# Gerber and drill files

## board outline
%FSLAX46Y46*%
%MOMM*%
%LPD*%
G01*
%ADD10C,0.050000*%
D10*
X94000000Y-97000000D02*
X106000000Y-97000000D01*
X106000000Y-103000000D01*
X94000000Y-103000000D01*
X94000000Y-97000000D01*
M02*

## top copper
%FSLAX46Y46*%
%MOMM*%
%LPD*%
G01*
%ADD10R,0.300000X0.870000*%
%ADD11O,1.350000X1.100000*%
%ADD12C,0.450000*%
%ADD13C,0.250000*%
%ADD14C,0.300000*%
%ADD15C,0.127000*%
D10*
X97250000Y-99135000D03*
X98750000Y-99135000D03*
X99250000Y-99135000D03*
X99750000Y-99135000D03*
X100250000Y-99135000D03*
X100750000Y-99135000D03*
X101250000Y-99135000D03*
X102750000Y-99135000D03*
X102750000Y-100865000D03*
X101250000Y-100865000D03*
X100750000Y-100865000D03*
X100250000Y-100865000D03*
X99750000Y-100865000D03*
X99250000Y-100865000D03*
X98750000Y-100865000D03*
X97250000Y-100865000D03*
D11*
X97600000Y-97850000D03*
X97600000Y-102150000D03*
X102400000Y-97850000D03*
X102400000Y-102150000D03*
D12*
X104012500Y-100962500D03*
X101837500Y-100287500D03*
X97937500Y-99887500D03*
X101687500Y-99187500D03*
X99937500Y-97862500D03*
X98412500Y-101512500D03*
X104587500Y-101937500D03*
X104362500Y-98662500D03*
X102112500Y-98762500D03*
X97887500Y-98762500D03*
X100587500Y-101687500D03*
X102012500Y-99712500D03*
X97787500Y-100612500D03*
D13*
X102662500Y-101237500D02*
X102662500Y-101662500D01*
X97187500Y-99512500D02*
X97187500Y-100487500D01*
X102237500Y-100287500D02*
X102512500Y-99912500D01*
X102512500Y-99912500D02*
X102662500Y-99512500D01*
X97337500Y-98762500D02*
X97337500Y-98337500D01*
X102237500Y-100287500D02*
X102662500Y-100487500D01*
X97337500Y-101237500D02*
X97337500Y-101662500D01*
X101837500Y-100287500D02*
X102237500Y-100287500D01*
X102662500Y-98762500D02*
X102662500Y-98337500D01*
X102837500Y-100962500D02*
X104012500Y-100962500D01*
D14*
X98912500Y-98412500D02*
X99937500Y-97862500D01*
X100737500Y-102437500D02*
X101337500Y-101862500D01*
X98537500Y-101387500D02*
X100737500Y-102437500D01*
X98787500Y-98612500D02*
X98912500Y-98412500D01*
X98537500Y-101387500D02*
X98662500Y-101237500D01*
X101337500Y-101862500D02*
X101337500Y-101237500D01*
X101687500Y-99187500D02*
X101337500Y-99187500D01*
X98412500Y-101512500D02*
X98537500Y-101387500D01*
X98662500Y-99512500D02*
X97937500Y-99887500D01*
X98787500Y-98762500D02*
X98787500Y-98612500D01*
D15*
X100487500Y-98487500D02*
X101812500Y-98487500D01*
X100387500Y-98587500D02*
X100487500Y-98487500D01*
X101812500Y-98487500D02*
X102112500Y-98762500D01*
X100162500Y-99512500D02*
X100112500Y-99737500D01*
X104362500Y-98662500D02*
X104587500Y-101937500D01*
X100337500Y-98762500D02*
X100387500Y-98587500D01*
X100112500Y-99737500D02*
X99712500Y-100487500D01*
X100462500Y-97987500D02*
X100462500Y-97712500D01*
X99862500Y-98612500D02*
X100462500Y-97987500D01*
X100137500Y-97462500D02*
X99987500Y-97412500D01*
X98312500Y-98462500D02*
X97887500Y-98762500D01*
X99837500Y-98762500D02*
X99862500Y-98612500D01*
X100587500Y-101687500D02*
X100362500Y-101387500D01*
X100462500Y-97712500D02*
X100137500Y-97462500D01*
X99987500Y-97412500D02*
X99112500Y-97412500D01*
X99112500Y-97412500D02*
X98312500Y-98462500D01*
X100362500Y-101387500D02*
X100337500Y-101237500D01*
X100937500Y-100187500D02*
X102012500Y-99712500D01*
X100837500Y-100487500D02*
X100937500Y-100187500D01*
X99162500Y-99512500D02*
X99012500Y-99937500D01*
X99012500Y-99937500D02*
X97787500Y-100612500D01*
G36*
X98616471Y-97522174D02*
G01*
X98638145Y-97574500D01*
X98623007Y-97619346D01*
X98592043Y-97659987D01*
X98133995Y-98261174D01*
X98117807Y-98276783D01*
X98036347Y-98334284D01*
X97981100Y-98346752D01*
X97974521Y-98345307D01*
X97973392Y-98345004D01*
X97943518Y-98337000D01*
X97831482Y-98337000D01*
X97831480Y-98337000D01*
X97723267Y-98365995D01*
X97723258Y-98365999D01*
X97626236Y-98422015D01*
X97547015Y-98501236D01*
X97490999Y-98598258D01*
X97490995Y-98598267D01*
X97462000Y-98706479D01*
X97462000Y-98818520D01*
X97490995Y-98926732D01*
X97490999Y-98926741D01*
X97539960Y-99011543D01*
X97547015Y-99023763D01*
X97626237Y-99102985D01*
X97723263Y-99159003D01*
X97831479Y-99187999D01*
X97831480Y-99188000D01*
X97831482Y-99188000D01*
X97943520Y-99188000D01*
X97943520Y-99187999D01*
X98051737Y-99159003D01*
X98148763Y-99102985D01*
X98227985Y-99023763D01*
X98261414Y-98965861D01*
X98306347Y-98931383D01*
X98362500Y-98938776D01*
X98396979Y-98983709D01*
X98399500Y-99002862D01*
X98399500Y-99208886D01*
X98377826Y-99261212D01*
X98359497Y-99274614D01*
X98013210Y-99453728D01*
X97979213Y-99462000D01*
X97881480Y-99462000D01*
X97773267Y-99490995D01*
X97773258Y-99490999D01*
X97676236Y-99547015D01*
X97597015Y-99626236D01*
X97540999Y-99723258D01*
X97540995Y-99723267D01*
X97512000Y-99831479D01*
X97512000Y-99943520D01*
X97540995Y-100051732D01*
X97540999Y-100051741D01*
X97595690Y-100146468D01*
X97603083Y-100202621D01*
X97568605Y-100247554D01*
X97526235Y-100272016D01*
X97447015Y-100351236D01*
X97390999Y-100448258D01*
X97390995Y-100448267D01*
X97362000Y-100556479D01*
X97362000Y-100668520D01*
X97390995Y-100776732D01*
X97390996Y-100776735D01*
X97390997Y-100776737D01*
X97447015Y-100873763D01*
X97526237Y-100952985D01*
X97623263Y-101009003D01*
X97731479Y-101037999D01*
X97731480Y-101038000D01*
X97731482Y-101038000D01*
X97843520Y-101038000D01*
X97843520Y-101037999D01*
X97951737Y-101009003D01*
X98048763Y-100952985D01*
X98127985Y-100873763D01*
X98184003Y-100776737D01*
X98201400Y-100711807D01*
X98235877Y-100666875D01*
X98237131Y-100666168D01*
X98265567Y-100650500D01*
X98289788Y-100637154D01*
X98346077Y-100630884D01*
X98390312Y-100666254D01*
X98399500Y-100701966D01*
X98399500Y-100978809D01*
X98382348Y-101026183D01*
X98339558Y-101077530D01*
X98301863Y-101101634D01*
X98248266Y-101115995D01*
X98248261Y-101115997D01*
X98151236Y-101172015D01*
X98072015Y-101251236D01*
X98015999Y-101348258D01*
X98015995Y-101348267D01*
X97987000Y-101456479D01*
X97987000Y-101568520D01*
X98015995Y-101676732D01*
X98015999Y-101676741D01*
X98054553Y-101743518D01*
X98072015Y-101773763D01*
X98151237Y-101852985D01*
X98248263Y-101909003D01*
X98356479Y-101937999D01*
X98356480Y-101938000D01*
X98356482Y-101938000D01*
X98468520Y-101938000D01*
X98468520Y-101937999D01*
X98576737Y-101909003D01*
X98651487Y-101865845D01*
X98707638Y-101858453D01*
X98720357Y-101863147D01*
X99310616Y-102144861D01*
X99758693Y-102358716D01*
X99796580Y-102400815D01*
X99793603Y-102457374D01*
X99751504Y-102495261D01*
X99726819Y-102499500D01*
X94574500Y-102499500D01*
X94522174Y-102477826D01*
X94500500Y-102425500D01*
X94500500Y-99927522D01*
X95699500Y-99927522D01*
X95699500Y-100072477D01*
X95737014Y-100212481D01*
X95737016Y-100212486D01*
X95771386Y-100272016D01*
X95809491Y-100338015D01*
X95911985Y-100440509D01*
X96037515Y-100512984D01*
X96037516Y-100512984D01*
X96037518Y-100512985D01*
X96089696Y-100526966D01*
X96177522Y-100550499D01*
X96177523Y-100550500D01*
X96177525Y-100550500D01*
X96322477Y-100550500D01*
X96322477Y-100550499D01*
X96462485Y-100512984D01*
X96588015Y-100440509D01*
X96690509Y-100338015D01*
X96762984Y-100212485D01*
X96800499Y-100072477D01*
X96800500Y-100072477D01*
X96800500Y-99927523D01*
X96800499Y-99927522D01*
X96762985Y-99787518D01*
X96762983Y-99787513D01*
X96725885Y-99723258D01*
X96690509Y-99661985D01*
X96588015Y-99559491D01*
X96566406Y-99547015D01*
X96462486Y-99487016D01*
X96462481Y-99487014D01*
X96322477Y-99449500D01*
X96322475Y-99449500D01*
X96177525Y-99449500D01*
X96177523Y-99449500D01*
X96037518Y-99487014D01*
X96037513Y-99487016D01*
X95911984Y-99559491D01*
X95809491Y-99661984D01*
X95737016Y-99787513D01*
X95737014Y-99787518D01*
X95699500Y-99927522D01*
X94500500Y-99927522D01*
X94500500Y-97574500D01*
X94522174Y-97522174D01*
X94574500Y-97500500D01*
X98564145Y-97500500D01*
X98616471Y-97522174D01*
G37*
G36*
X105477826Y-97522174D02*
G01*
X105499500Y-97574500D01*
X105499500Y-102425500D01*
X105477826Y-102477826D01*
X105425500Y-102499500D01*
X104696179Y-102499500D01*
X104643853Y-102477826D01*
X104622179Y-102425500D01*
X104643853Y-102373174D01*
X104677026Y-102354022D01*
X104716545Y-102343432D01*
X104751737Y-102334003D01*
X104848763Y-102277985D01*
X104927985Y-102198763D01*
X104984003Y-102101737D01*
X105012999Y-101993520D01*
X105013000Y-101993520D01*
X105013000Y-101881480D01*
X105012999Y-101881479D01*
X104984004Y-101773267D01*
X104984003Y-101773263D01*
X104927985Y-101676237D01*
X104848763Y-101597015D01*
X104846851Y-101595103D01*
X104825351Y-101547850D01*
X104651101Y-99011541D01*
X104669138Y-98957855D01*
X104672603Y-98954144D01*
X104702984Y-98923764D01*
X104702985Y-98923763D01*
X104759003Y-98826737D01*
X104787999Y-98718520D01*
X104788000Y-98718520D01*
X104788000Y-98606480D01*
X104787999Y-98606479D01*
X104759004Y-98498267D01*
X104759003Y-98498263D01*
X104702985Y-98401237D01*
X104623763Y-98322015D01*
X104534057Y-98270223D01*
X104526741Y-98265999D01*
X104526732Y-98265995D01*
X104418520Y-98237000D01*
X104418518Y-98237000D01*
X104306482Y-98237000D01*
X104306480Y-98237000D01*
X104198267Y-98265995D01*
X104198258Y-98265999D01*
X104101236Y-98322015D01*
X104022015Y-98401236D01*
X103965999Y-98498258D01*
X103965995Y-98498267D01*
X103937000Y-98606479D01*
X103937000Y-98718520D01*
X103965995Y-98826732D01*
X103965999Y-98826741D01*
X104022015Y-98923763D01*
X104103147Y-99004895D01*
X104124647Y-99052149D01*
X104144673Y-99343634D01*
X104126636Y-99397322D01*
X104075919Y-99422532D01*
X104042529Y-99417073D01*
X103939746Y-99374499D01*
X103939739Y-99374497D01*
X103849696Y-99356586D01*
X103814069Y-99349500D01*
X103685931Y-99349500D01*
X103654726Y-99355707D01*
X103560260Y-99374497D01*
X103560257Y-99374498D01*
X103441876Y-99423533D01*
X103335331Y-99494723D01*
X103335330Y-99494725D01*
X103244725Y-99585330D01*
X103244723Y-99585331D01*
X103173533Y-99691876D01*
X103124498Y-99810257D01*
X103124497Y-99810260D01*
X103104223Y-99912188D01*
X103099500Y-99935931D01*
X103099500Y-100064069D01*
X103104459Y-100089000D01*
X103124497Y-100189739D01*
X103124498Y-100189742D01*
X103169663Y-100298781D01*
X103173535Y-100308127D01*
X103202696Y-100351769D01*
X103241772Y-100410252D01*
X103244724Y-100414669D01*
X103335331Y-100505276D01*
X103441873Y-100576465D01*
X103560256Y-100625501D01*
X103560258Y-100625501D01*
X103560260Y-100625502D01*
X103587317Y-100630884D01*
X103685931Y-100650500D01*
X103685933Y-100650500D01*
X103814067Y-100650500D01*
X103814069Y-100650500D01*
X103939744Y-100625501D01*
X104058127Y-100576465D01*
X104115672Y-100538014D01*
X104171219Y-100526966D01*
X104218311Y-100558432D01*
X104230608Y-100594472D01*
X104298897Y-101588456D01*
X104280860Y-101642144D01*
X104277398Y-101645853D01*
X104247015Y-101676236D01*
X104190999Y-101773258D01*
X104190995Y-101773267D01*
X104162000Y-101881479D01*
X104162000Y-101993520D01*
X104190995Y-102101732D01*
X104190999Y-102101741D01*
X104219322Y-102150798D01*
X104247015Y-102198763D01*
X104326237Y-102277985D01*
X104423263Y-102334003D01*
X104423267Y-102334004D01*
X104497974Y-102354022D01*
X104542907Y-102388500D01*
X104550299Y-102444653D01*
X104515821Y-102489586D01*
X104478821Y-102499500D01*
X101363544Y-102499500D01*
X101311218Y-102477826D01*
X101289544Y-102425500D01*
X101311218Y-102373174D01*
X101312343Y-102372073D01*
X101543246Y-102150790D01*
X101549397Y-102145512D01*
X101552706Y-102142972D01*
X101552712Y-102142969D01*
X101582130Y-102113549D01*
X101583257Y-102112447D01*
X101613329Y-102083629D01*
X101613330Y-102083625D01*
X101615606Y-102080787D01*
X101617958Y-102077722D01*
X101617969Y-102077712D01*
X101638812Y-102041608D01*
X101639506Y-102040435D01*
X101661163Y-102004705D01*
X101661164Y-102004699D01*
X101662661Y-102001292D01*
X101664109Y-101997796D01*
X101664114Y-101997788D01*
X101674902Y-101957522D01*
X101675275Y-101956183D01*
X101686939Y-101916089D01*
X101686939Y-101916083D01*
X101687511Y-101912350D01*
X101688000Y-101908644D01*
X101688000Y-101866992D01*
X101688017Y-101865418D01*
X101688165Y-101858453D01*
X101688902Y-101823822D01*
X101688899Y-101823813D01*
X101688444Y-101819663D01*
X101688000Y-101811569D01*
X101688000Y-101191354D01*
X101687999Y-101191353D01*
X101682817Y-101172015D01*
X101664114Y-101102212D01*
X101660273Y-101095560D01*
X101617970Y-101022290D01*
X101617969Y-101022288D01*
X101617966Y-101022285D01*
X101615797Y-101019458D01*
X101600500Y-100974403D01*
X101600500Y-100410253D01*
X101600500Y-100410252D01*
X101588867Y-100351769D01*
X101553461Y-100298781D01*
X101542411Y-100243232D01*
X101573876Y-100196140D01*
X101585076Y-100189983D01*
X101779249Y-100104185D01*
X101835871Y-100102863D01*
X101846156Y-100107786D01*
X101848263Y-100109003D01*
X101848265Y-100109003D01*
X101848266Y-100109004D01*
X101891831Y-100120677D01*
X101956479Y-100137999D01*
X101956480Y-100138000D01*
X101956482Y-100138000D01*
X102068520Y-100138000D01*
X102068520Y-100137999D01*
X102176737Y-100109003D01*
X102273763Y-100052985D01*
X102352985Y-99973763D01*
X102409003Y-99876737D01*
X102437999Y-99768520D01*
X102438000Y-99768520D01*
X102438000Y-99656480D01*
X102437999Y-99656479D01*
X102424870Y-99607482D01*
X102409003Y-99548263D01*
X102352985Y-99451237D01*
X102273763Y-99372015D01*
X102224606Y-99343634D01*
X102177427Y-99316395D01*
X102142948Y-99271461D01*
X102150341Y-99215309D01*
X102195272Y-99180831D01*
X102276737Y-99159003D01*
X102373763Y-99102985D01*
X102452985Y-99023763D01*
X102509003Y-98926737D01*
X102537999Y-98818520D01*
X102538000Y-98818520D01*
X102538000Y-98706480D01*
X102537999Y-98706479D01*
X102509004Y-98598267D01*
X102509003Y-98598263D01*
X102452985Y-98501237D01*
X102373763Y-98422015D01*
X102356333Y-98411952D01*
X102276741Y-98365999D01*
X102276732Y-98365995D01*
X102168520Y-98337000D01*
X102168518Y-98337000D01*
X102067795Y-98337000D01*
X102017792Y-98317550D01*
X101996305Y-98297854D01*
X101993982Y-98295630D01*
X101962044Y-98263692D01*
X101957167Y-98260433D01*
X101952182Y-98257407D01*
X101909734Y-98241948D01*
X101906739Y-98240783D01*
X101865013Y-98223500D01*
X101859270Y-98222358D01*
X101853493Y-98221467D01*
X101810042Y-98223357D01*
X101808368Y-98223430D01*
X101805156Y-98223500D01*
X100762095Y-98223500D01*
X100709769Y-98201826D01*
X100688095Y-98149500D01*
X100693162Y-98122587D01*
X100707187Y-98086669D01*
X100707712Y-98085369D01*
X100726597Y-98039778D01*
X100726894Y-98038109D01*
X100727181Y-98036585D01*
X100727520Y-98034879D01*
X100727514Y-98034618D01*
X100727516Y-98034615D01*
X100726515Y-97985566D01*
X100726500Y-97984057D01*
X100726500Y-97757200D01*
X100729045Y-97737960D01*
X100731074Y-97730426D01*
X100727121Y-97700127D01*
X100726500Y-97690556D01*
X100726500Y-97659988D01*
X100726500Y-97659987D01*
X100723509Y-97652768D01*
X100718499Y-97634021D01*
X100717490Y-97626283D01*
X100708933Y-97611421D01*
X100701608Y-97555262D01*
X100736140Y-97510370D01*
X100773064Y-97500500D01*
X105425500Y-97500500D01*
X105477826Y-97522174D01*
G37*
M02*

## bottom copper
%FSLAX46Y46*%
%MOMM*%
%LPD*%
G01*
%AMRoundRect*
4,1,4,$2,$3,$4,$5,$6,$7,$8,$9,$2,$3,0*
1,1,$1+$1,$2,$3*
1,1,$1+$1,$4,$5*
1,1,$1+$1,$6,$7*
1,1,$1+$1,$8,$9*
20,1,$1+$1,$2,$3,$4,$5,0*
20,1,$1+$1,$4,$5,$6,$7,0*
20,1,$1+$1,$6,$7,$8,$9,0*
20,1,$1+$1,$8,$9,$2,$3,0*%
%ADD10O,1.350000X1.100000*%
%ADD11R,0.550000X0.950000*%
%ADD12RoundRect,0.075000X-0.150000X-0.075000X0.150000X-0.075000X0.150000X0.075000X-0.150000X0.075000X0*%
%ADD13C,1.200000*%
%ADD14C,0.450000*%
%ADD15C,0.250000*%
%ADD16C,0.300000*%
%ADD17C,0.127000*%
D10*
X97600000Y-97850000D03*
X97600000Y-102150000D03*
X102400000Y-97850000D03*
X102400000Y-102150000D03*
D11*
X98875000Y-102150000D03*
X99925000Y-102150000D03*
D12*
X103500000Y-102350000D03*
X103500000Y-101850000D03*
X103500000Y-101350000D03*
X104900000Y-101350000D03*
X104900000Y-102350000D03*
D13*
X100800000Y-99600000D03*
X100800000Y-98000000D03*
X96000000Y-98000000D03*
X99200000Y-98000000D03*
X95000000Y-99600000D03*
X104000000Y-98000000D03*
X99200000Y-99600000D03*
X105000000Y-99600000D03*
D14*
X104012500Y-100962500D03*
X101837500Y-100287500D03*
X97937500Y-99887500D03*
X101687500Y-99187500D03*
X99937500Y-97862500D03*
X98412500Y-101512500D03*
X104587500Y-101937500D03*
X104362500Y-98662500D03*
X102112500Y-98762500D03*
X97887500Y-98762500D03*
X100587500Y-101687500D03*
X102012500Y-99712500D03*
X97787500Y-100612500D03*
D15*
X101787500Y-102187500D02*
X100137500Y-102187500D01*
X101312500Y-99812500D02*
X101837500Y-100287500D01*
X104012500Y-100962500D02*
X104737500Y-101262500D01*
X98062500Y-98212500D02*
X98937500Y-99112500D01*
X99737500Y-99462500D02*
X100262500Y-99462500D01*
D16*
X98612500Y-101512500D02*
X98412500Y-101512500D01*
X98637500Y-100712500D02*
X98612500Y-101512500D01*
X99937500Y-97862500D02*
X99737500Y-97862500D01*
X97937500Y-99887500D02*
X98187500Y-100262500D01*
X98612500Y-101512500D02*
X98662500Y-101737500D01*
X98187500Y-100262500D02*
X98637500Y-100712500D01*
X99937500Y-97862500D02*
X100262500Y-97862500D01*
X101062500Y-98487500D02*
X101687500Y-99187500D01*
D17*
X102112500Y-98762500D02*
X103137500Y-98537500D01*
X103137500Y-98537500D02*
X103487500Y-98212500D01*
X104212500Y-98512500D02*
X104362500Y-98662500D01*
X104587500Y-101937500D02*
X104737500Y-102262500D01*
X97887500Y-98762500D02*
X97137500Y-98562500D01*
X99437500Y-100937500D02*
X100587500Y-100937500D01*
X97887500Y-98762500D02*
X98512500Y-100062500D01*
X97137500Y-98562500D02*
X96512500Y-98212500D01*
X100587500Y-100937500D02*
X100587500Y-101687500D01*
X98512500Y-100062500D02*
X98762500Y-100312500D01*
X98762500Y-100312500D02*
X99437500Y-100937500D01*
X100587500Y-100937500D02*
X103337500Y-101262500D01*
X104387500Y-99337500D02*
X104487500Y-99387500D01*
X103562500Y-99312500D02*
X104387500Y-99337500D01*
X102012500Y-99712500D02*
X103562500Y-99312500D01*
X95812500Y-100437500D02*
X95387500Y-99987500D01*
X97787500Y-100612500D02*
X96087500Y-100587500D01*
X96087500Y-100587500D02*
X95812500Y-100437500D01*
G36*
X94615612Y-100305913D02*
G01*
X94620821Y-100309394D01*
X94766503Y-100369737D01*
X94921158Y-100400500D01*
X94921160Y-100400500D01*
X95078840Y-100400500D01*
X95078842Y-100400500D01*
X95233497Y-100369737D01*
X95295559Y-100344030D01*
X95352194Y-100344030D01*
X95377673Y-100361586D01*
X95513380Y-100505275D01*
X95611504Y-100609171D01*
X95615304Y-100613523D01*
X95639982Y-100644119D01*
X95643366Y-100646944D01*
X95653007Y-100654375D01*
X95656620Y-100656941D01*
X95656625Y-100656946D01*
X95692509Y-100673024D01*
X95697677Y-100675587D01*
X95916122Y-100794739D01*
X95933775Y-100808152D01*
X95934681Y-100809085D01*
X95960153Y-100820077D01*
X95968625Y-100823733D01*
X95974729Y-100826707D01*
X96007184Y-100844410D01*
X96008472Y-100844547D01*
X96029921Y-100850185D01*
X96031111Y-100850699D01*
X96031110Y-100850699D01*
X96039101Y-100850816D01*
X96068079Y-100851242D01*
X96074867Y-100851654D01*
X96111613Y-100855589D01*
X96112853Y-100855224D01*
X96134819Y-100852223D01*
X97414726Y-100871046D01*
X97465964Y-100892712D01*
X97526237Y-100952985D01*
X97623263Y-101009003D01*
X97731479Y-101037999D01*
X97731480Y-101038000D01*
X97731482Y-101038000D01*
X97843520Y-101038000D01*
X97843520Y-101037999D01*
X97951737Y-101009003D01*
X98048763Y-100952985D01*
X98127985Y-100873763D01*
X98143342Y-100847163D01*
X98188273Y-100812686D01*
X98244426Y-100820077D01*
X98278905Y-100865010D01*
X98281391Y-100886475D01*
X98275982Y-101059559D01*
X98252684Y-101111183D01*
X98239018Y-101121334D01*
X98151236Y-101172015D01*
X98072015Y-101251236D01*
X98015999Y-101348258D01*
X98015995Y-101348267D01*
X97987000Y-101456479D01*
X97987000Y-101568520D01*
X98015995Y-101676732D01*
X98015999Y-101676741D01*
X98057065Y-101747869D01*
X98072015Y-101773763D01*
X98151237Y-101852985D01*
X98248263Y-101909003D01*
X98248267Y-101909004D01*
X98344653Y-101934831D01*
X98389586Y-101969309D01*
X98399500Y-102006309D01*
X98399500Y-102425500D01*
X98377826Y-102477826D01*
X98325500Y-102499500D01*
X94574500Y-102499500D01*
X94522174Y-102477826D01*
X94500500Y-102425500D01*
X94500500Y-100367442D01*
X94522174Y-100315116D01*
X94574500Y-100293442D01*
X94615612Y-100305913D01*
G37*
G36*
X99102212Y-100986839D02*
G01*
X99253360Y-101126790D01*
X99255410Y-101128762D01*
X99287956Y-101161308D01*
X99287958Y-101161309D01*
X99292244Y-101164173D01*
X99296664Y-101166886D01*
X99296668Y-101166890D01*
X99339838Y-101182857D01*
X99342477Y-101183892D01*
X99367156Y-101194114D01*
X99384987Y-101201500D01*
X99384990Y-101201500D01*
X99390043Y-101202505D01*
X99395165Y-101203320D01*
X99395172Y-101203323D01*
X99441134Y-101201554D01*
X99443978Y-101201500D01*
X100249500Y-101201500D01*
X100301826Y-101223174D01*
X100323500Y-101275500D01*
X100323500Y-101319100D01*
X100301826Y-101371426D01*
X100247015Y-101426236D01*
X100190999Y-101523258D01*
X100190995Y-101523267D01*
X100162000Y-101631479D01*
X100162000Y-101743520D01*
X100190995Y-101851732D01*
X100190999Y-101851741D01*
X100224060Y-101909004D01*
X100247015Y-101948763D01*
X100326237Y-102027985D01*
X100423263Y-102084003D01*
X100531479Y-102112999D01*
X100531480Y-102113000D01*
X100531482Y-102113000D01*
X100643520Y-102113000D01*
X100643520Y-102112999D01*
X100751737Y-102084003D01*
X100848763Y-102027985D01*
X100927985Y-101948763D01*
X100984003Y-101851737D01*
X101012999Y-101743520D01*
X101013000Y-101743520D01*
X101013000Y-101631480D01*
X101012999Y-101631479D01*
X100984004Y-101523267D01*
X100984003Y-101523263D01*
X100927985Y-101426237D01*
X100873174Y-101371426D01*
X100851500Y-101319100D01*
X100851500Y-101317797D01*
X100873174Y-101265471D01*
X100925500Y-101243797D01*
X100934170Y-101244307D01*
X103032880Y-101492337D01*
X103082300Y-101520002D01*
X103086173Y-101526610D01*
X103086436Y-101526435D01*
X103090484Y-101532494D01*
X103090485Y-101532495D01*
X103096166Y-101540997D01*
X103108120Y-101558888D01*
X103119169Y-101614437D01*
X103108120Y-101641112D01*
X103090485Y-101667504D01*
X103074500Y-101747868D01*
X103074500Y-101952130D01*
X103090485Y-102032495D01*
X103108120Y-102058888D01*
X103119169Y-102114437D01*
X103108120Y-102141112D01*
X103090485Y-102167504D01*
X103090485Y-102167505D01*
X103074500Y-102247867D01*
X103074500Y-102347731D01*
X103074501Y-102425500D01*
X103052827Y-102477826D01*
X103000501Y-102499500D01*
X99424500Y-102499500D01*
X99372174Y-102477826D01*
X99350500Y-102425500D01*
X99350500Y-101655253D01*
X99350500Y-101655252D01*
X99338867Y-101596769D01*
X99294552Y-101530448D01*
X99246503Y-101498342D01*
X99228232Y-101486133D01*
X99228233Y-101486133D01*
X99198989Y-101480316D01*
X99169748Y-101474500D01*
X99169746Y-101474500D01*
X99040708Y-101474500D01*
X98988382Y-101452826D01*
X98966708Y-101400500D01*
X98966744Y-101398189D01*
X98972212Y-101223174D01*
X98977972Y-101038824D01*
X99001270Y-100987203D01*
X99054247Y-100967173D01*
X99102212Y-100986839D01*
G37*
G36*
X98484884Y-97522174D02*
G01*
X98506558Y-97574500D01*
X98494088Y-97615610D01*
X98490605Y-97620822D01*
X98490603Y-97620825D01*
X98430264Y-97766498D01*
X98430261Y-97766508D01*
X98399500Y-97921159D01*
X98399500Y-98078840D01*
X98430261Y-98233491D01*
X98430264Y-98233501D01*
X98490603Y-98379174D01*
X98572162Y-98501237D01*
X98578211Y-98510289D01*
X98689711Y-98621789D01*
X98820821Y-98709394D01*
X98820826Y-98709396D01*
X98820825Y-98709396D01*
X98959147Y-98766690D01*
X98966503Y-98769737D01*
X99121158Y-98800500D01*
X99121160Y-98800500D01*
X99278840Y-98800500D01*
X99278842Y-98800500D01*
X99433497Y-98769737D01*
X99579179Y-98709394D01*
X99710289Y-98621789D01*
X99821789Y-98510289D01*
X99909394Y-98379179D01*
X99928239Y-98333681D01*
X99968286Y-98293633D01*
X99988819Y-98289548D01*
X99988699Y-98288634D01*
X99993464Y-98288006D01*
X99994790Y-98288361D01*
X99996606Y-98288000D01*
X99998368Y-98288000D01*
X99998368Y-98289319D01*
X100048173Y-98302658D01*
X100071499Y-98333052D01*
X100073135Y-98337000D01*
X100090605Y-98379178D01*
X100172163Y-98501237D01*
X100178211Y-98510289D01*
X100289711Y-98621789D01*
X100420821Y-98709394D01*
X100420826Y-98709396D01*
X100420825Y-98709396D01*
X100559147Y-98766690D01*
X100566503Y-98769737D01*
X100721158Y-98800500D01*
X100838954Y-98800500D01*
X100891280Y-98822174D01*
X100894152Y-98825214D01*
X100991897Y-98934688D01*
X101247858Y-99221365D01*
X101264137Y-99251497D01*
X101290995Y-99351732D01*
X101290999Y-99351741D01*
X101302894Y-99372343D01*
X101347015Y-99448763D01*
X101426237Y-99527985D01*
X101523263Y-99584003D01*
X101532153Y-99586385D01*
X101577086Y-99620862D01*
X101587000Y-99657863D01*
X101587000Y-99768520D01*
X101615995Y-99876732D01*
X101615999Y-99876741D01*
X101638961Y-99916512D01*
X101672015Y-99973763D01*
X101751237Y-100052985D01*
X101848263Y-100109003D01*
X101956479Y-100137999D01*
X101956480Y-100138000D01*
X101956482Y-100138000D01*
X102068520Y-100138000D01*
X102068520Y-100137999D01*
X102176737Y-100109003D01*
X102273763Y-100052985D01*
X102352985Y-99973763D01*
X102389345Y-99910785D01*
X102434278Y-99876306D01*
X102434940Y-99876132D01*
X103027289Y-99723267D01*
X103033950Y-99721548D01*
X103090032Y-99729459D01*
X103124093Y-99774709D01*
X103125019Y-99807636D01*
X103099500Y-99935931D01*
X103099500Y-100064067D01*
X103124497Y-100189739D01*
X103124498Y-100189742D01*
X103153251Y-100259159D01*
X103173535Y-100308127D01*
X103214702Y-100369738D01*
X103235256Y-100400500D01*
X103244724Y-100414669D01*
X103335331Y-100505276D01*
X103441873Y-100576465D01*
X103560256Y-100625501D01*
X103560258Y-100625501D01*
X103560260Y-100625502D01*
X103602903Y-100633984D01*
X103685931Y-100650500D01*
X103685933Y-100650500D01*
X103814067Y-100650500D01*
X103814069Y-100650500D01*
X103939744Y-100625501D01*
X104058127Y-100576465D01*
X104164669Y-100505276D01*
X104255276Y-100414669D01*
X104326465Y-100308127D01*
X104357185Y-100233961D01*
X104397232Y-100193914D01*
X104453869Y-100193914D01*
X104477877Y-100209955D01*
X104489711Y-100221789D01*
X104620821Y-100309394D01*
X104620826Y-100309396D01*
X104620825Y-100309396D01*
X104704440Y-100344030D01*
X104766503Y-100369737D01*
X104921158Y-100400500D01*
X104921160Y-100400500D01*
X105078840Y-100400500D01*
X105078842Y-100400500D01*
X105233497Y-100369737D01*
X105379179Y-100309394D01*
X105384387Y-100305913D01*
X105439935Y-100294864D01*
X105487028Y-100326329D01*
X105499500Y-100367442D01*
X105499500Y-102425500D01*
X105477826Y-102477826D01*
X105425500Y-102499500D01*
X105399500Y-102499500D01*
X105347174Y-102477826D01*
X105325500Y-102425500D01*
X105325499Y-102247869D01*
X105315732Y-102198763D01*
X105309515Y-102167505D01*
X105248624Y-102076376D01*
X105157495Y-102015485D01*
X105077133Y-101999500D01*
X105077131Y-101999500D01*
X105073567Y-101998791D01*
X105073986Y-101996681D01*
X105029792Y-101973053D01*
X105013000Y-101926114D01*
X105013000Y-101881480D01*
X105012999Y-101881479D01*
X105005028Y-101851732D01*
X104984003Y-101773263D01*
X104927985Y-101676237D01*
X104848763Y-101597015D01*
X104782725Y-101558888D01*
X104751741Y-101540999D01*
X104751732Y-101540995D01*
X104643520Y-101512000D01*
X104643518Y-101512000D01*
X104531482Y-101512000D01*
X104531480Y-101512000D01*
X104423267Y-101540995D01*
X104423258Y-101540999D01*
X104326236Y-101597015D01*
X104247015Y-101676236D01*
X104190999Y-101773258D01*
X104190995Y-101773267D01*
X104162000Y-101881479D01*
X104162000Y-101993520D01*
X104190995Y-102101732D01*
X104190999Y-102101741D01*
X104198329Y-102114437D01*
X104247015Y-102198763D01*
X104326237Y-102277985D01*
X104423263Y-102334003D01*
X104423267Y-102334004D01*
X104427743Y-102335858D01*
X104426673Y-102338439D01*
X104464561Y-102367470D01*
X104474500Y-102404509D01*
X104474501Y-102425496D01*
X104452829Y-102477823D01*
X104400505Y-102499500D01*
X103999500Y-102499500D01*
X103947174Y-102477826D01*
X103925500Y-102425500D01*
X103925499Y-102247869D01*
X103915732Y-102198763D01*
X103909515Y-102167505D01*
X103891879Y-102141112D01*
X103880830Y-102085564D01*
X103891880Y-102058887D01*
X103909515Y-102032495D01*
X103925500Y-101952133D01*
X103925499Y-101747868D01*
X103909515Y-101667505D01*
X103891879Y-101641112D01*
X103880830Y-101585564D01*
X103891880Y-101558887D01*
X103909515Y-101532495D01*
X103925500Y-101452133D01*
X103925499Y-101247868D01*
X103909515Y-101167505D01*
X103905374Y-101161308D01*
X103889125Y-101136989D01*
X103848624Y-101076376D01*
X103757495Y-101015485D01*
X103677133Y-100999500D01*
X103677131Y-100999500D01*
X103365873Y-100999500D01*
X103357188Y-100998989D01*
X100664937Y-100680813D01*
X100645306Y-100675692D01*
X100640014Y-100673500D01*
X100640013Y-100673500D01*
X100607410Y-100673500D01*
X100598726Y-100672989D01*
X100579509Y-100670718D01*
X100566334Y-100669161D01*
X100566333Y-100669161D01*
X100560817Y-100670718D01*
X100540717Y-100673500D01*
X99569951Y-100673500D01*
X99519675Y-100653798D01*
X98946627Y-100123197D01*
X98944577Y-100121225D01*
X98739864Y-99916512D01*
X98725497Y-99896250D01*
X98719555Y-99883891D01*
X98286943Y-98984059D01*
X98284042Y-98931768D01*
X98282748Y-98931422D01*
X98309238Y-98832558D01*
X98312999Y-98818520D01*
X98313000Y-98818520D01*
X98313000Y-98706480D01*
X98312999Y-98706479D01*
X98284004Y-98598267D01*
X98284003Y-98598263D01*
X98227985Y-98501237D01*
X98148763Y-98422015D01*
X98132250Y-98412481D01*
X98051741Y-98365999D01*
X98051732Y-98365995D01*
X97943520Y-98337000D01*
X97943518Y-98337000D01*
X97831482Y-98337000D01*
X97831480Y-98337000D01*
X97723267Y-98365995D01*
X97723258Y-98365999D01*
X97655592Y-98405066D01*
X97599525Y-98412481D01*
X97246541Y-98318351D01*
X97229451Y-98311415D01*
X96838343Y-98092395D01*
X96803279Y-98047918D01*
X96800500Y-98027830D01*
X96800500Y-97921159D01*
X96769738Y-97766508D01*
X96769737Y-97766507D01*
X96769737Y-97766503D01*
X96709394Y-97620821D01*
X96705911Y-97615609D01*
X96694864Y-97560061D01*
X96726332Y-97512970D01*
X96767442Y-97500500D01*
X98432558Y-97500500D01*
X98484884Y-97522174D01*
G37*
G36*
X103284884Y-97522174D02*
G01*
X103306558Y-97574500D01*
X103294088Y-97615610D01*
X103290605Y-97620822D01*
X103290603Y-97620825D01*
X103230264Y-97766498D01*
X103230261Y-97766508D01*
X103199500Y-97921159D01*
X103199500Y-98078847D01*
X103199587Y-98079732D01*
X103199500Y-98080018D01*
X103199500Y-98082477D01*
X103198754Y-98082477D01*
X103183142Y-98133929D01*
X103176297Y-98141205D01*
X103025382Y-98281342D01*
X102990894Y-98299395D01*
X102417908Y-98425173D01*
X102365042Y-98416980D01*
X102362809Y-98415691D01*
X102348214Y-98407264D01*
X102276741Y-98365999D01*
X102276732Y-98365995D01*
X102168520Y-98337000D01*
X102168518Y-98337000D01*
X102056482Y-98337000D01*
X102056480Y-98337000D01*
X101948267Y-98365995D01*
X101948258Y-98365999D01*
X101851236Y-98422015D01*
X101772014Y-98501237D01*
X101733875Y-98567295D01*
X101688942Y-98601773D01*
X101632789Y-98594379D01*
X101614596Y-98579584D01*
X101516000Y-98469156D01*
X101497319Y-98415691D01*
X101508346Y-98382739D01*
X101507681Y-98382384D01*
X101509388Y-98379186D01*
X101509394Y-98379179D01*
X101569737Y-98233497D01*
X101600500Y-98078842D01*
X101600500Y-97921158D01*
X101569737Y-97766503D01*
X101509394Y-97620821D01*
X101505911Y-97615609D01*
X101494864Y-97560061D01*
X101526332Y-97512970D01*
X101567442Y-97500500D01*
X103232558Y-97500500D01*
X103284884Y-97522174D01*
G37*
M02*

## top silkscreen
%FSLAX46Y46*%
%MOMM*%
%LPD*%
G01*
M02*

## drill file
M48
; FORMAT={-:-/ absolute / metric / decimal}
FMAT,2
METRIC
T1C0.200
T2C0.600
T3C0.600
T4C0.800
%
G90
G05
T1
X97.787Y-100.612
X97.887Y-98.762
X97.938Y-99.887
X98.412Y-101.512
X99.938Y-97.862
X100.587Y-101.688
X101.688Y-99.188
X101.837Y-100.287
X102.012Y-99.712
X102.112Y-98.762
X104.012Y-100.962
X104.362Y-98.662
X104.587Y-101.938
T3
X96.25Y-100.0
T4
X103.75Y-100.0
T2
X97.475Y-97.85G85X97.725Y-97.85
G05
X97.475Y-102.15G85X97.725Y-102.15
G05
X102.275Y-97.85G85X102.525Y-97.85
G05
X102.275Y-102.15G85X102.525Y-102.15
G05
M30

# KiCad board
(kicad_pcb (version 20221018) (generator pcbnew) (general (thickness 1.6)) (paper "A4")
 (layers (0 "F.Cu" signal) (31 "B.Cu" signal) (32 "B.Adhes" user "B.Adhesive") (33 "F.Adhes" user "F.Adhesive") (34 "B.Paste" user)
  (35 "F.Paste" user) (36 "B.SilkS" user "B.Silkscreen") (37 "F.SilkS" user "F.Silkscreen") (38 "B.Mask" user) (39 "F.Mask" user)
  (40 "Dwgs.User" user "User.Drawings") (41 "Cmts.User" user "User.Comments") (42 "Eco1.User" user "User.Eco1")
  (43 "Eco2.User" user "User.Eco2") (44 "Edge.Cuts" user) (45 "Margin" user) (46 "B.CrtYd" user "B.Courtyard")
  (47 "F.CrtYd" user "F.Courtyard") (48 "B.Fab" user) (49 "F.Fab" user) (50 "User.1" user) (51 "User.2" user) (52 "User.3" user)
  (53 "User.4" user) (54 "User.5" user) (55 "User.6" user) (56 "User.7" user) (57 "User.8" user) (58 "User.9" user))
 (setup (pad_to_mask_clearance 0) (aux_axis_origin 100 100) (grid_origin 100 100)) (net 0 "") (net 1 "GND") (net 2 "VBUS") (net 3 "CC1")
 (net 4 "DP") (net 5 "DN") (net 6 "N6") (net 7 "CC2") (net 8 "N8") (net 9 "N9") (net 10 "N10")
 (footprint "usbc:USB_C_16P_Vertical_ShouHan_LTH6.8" (layer "F.Cu") (at 100 100)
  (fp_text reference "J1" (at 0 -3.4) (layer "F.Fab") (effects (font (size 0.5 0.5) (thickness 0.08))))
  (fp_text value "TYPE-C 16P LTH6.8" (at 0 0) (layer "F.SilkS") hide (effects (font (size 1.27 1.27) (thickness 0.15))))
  (pad "" np_thru_hole circle (at -3.75 0) (size 0.6 0.6) (drill 0.6) (layers "F&B.Cu" "*.Mask"))
  (pad "" np_thru_hole circle (at 3.75 0) (size 0.8 0.8) (drill 0.8) (layers "F&B.Cu" "*.Mask"))
  (pad "A1" smd rect (at -2.75 -0.865) (size 0.3 0.87) (layers "F.Cu" "F.Paste" "F.Mask") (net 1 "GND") (thermal_bridge_angle 45))
  (pad "A4" smd rect (at -1.25 -0.865) (size 0.3 0.87) (layers "F.Cu" "F.Paste" "F.Mask") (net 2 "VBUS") (thermal_bridge_angle 45))
  (pad "A5" smd rect (at -0.75 -0.865) (size 0.3 0.87) (layers "F.Cu" "F.Paste" "F.Mask") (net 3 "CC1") (thermal_bridge_angle 45))
  (pad "A6" smd rect (at -0.25 -0.865) (size 0.3 0.87) (layers "F.Cu" "F.Paste" "F.Mask") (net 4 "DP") (thermal_bridge_angle 45))
  (pad "A7" smd rect (at 0.25 -0.865) (size 0.3 0.87) (layers "F.Cu" "F.Paste" "F.Mask") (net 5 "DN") (thermal_bridge_angle 45))
  (pad "A8" smd rect (at 0.75 -0.865) (size 0.3 0.87) (layers "F.Cu" "F.Paste" "F.Mask") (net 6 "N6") (thermal_bridge_angle 45))
  (pad "A9" smd rect (at 1.25 -0.865) (size 0.3 0.87) (layers "F.Cu" "F.Paste" "F.Mask") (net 2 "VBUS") (thermal_bridge_angle 45))
  (pad "A12" smd rect (at 2.75 -0.865) (size 0.3 0.87) (layers "F.Cu" "F.Paste" "F.Mask") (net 1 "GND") (thermal_bridge_angle 45))
  (pad "B1" smd rect (at 2.75 0.865) (size 0.3 0.87) (layers "F.Cu" "F.Paste" "F.Mask") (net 1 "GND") (thermal_bridge_angle 45))
  (pad "B4" smd rect (at 1.25 0.865) (size 0.3 0.87) (layers "F.Cu" "F.Paste" "F.Mask") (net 2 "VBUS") (thermal_bridge_angle 45))
  (pad "B5" smd rect (at 0.75 0.865) (size 0.3 0.87) (layers "F.Cu" "F.Paste" "F.Mask") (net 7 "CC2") (thermal_bridge_angle 45))
  (pad "B6" smd rect (at 0.25 0.865) (size 0.3 0.87) (layers "F.Cu" "F.Paste" "F.Mask") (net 4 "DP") (thermal_bridge_angle 45))
  (pad "B7" smd rect (at -0.25 0.865) (size 0.3 0.87) (layers "F.Cu" "F.Paste" "F.Mask") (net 5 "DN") (thermal_bridge_angle 45))
  (pad "B8" smd rect (at -0.75 0.865) (size 0.3 0.87) (layers "F.Cu" "F.Paste" "F.Mask") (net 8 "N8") (thermal_bridge_angle 45))
  (pad "B9" smd rect (at -1.25 0.865) (size 0.3 0.87) (layers "F.Cu" "F.Paste" "F.Mask") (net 2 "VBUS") (thermal_bridge_angle 45))
  (pad "B12" smd rect (at -2.75 0.865) (size 0.3 0.87) (layers "F.Cu" "F.Paste" "F.Mask") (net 1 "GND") (thermal_bridge_angle 45))
  (pad "S" thru_hole oval (at -2.4 -2.15) (size 1.35 1.1) (drill oval 0.85 0.6) (layers "*.Cu" "*.Mask") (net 1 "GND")
   (thermal_bridge_angle 45))
  (pad "S" thru_hole oval (at -2.4 2.15) (size 1.35 1.1) (drill oval 0.85 0.6) (layers "*.Cu" "*.Mask") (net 1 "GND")
   (thermal_bridge_angle 45))
  (pad "S" thru_hole oval (at 2.4 -2.15) (size 1.35 1.1) (drill oval 0.85 0.6) (layers "*.Cu" "*.Mask") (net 1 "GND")
   (thermal_bridge_angle 45))
  (pad "S" thru_hole oval (at 2.4 2.15) (size 1.35 1.1) (drill oval 0.85 0.6) (layers "*.Cu" "*.Mask") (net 1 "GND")
   (thermal_bridge_angle 45)))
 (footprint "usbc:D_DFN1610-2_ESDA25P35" (layer "B.Cu") (at 99.4 102.15)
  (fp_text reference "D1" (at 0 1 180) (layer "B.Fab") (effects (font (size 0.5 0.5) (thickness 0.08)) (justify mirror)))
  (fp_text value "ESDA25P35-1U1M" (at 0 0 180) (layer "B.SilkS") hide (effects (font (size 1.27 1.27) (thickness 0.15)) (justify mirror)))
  (pad "1" smd rect (at -0.525 0) (size 0.55 0.95) (layers "B.Cu" "B.Paste" "B.Mask") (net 2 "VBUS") (thermal_bridge_angle 45))
  (pad "2" smd rect (at 0.525 0) (size 0.55 0.95) (layers "B.Cu" "B.Paste" "B.Mask") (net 1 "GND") (thermal_bridge_angle 45)))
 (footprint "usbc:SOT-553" (layer "B.Cu") (at 104.2 101.85)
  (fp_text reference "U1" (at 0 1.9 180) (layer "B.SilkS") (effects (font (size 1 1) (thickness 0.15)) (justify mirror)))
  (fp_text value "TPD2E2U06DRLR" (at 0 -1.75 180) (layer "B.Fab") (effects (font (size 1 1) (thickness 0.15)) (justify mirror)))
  (pad "1" smd roundrect (at -0.7 0.5) (size 0.45 0.3) (layers "B.Cu" "B.Paste" "B.Mask") (roundrect_rratio 0.25) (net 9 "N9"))
  (pad "2" smd roundrect (at -0.7 0) (size 0.45 0.3) (layers "B.Cu" "B.Paste" "B.Mask") (roundrect_rratio 0.25) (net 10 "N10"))
  (pad "3" smd roundrect (at -0.7 -0.5) (size 0.45 0.3) (layers "B.Cu" "B.Paste" "B.Mask") (roundrect_rratio 0.25) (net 4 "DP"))
  (pad "4" smd roundrect (at 0.7 -0.5) (size 0.45 0.3) (layers "B.Cu" "B.Paste" "B.Mask") (roundrect_rratio 0.25) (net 1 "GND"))
  (pad "5" smd roundrect (at 0.7 0.5) (size 0.45 0.3) (layers "B.Cu" "B.Paste" "B.Mask") (roundrect_rratio 0.25) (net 5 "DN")))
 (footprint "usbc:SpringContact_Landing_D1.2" (layer "B.Cu") (at 100.8 99.6)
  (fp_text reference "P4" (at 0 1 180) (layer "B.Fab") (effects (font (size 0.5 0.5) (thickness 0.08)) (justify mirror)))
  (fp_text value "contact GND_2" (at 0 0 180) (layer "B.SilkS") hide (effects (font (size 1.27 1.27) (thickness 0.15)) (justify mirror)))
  (pad "1" smd circle (at 0 0) (size 1.2 1.2) (layers "B.Cu" "B.Mask") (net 1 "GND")))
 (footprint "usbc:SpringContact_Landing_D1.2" (layer "B.Cu") (at 100.8 98)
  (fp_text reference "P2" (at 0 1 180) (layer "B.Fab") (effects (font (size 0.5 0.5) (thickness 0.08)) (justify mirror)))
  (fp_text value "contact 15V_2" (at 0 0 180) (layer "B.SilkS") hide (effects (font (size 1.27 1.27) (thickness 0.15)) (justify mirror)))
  (pad "1" smd circle (at 0 0) (size 1.2 1.2) (layers "B.Cu" "B.Mask") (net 2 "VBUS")))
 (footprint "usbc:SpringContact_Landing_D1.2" (layer "B.Cu") (at 96 98)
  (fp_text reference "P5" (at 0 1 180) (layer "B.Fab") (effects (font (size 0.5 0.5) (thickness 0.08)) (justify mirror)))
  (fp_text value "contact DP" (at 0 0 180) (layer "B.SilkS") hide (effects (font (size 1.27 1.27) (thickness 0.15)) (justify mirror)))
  (pad "1" smd circle (at 0 0) (size 1.2 1.2) (layers "B.Cu" "B.Mask") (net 4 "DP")))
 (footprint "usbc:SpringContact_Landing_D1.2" (layer "B.Cu") (at 99.2 98)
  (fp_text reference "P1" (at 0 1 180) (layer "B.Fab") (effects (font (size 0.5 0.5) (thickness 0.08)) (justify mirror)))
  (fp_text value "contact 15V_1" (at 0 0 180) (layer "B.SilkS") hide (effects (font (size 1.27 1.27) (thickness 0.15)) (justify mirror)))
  (pad "1" smd circle (at 0 0) (size 1.2 1.2) (layers "B.Cu" "B.Mask") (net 2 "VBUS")))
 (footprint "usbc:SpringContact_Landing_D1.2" (layer "B.Cu") (at 95 99.6)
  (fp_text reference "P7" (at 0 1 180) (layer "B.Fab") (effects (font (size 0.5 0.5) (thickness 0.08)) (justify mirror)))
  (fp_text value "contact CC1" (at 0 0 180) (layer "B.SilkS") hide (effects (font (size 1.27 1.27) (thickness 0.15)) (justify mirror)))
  (pad "1" smd circle (at 0 0) (size 1.2 1.2) (layers "B.Cu" "B.Mask") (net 3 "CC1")))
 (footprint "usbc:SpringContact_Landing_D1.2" (layer "B.Cu") (at 104 98)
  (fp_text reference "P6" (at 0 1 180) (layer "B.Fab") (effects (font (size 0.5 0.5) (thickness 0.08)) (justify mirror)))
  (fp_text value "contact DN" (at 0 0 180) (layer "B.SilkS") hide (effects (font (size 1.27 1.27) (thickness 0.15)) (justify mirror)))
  (pad "1" smd circle (at 0 0) (size 1.2 1.2) (layers "B.Cu" "B.Mask") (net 5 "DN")))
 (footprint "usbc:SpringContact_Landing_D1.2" (layer "B.Cu") (at 99.2 99.6)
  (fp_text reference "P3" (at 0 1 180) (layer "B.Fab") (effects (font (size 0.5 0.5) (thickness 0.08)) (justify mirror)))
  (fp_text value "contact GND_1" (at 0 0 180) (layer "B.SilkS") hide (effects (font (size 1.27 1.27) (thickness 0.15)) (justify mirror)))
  (pad "1" smd circle (at 0 0) (size 1.2 1.2) (layers "B.Cu" "B.Mask") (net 1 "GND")))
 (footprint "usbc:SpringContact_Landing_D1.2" (layer "B.Cu") (at 105 99.6)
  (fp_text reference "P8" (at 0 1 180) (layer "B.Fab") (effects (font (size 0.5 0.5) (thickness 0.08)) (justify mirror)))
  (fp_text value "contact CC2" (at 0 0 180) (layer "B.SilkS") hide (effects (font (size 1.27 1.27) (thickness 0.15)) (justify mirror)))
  (pad "1" smd circle (at 0 0) (size 1.2 1.2) (layers "B.Cu" "B.Mask") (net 7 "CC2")))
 (gr_rect (start 94 97) (end 106 103) (stroke (width 0.05) (type default)) (fill none) (layer "Edge.Cuts"))
 (segment (start 102.6625 101.2375) (end 102.6625 101.6625) (width 0.25) (layer "F.Cu") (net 1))
 (segment (start 97.1875 99.5125) (end 97.1875 100.4875) (width 0.25) (layer "F.Cu") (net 1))
 (segment (start 102.2375 100.2875) (end 102.5125 99.9125) (width 0.25) (layer "F.Cu") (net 1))
 (segment (start 102.5125 99.9125) (end 102.6625 99.5125) (width 0.25) (layer "F.Cu") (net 1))
 (segment (start 97.3375 98.7625) (end 97.3375 98.3375) (width 0.25) (layer "F.Cu") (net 1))
 (segment (start 102.2375 100.2875) (end 102.6625 100.4875) (width 0.25) (layer "F.Cu") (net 1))
 (segment (start 97.3375 101.2375) (end 97.3375 101.6625) (width 0.25) (layer "F.Cu") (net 1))
 (segment (start 101.8375 100.2875) (end 102.2375 100.2875) (width 0.25) (layer "F.Cu") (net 1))
 (segment (start 102.6625 98.7625) (end 102.6625 98.3375) (width 0.25) (layer "F.Cu") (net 1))
 (segment (start 102.8375 100.9625) (end 104.0125 100.9625) (width 0.25) (layer "F.Cu") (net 1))
 (via (at 104.0125 100.9625) (size 0.45) (drill 0.2) (layers "F.Cu" "B.Cu") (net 1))
 (via (at 101.8375 100.2875) (size 0.45) (drill 0.2) (layers "F.Cu" "B.Cu") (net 1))
 (segment (start 101.7875 102.1875) (end 100.1375 102.1875) (width 0.25) (layer "B.Cu") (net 1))
 (segment (start 101.3125 99.8125) (end 101.8375 100.2875) (width 0.25) (layer "B.Cu") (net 1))
 (segment (start 104.0125 100.9625) (end 104.7375 101.2625) (width 0.25) (layer "B.Cu") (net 1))
 (segment (start 98.0625 98.2125) (end 98.9375 99.1125) (width 0.25) (layer "B.Cu") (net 1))
 (segment (start 99.7375 99.4625) (end 100.2625 99.4625) (width 0.25) (layer "B.Cu") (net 1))
 (segment (start 98.9125 98.4125) (end 99.9375 97.8625) (width 0.3) (layer "F.Cu") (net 2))
 (segment (start 100.7375 102.4375) (end 101.3375 101.8625) (width 0.3) (layer "F.Cu") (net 2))
 (segment (start 98.5375 101.3875) (end 100.7375 102.4375) (width 0.3) (layer "F.Cu") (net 2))
 (segment (start 98.7875 98.6125) (end 98.9125 98.4125) (width 0.3) (layer "F.Cu") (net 2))
 (segment (start 98.5375 101.3875) (end 98.6625 101.2375) (width 0.3) (layer "F.Cu") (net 2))
 (segment (start 101.3375 101.8625) (end 101.3375 101.2375) (width 0.3) (layer "F.Cu") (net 2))
 (segment (start 101.6875 99.1875) (end 101.3375 99.1875) (width 0.3) (layer "F.Cu") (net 2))
 (segment (start 98.4125 101.5125) (end 98.5375 101.3875) (width 0.3) (layer "F.Cu") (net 2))
 (segment (start 98.6625 99.5125) (end 97.9375 99.8875) (width 0.3) (layer "F.Cu") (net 2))
 (segment (start 98.7875 98.7625) (end 98.7875 98.6125) (width 0.3) (layer "F.Cu") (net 2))
 (via (at 97.9375 99.8875) (size 0.45) (drill 0.2) (layers "F.Cu" "B.Cu") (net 2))
 (via (at 101.6875 99.1875) (size 0.45) (drill 0.2) (layers "F.Cu" "B.Cu") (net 2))
 (via (at 99.9375 97.8625) (size 0.45) (drill 0.2) (layers "F.Cu" "B.Cu") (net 2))
 (via (at 98.4125 101.5125) (size 0.45) (drill 0.2) (layers "F.Cu" "B.Cu") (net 2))
 (segment (start 98.6125 101.5125) (end 98.4125 101.5125) (width 0.3) (layer "B.Cu") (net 2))
 (segment (start 98.6375 100.7125) (end 98.6125 101.5125) (width 0.3) (layer "B.Cu") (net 2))
 (segment (start 99.9375 97.8625) (end 99.7375 97.8625) (width 0.3) (layer "B.Cu") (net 2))
 (segment (start 97.9375 99.8875) (end 98.1875 100.2625) (width 0.3) (layer "B.Cu") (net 2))
 (segment (start 98.6125 101.5125) (end 98.6625 101.7375) (width 0.3) (layer "B.Cu") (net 2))
 (segment (start 98.1875 100.2625) (end 98.6375 100.7125) (width 0.3) (layer "B.Cu") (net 2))
 (segment (start 99.9375 97.8625) (end 100.2625 97.8625) (width 0.3) (layer "B.Cu") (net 2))
 (segment (start 101.0625 98.4875) (end 101.6875 99.1875) (width 0.3) (layer "B.Cu") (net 2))
 (segment (start 100.4875 98.4875) (end 101.8125 98.4875) (width 0.127) (layer "F.Cu") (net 5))
 (segment (start 100.3875 98.5875) (end 100.4875 98.4875) (width 0.127) (layer "F.Cu") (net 5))
 (segment (start 101.8125 98.4875) (end 102.1125 98.7625) (width 0.127) (layer "F.Cu") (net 5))
 (segment (start 100.1625 99.5125) (end 100.1125 99.7375) (width 0.127) (layer "F.Cu") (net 5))
 (segment (start 104.3625 98.6625) (end 104.5875 101.9375) (width 0.127) (layer "F.Cu") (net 5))
 (segment (start 100.3375 98.7625) (end 100.3875 98.5875) (width 0.127) (layer "F.Cu") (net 5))
 (segment (start 100.1125 99.7375) (end 99.7125 100.4875) (width 0.127) (layer "F.Cu") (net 5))
 (via (at 104.5875 101.9375) (size 0.45) (drill 0.2) (layers "F.Cu" "B.Cu") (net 5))
 (via (at 104.3625 98.6625) (size 0.45) (drill 0.2) (layers "F.Cu" "B.Cu") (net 5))
 (via (at 102.1125 98.7625) (size 0.45) (drill 0.2) (layers "F.Cu" "B.Cu") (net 5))
 (segment (start 102.1125 98.7625) (end 103.1375 98.5375) (width 0.127) (layer "B.Cu") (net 5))
 (segment (start 103.1375 98.5375) (end 103.4875 98.2125) (width 0.127) (layer "B.Cu") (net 5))
 (segment (start 104.2125 98.5125) (end 104.3625 98.6625) (width 0.127) (layer "B.Cu") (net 5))
 (segment (start 104.5875 101.9375) (end 104.7375 102.2625) (width 0.127) (layer "B.Cu") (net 5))
 (segment (start 100.4625 97.9875) (end 100.4625 97.7125) (width 0.127) (layer "F.Cu") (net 4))
 (segment (start 99.8625 98.6125) (end 100.4625 97.9875) (width 0.127) (layer "F.Cu") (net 4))
 (segment (start 100.1375 97.4625) (end 99.9875 97.4125) (width 0.127) (layer "F.Cu") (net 4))
 (segment (start 98.3125 98.4625) (end 97.8875 98.7625) (width 0.127) (layer "F.Cu") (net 4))
 (segment (start 99.8375 98.7625) (end 99.8625 98.6125) (width 0.127) (layer "F.Cu") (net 4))
 (segment (start 100.5875 101.6875) (end 100.3625 101.3875) (width 0.127) (layer "F.Cu") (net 4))
 (segment (start 100.4625 97.7125) (end 100.1375 97.4625) (width 0.127) (layer "F.Cu") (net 4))
 (segment (start 99.9875 97.4125) (end 99.1125 97.4125) (width 0.127) (layer "F.Cu") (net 4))
 (segment (start 99.1125 97.4125) (end 98.3125 98.4625) (width 0.127) (layer "F.Cu") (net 4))
 (segment (start 100.3625 101.3875) (end 100.3375 101.2375) (width 0.127) (layer "F.Cu") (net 4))
 (via (at 97.8875 98.7625) (size 0.45) (drill 0.2) (layers "F.Cu" "B.Cu") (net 4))
 (via (at 100.5875 101.6875) (size 0.45) (drill 0.2) (layers "F.Cu" "B.Cu") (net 4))
 (segment (start 97.8875 98.7625) (end 97.1375 98.5625) (width 0.127) (layer "B.Cu") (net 4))
 (segment (start 99.4375 100.9375) (end 100.5875 100.9375) (width 0.127) (layer "B.Cu") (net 4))
 (segment (start 97.8875 98.7625) (end 98.5125 100.0625) (width 0.127) (layer "B.Cu") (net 4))
 (segment (start 97.1375 98.5625) (end 96.5125 98.2125) (width 0.127) (layer "B.Cu") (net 4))
 (segment (start 100.5875 100.9375) (end 100.5875 101.6875) (width 0.127) (layer "B.Cu") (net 4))
 (segment (start 98.5125 100.0625) (end 98.7625 100.3125) (width 0.127) (layer "B.Cu") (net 4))
 (segment (start 98.7625 100.3125) (end 99.4375 100.9375) (width 0.127) (layer "B.Cu") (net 4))
 (segment (start 100.5875 100.9375) (end 103.3375 101.2625) (width 0.127) (layer "B.Cu") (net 4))
 (segment (start 100.9375 100.1875) (end 102.0125 99.7125) (width 0.127) (layer "F.Cu") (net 7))
 (segment (start 100.8375 100.4875) (end 100.9375 100.1875) (width 0.127) (layer "F.Cu") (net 7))
 (via (at 102.0125 99.7125) (size 0.45) (drill 0.2) (layers "F.Cu" "B.Cu") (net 7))
 (segment (start 104.3875 99.3375) (end 104.4875 99.3875) (width 0.127) (layer "B.Cu") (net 7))
 (segment (start 103.5625 99.3125) (end 104.3875 99.3375) (width 0.127) (layer "B.Cu") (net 7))
 (segment (start 102.0125 99.7125) (end 103.5625 99.3125) (width 0.127) (layer "B.Cu") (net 7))
 (segment (start 99.1625 99.5125) (end 99.0125 99.9375) (width 0.127) (layer "F.Cu") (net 3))
 (segment (start 99.0125 99.9375) (end 97.7875 100.6125) (width 0.127) (layer "F.Cu") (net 3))
 (via (at 97.7875 100.6125) (size 0.45) (drill 0.2) (layers "F.Cu" "B.Cu") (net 3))
 (segment (start 95.8125 100.4375) (end 95.3875 99.9875) (width 0.127) (layer "B.Cu") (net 3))
 (segment (start 97.7875 100.6125) (end 96.0875 100.5875) (width 0.127) (layer "B.Cu") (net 3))
 (segment (start 96.0875 100.5875) (end 95.8125 100.4375) (width 0.127) (layer "B.Cu") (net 3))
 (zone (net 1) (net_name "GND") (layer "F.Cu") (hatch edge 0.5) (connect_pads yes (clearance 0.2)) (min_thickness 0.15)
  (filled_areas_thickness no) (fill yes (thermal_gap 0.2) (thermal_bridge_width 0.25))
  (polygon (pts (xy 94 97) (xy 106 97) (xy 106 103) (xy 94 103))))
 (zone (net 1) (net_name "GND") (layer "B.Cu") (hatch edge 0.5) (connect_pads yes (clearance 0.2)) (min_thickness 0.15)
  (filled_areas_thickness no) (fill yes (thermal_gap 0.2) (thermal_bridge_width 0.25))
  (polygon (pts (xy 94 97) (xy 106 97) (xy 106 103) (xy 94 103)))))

